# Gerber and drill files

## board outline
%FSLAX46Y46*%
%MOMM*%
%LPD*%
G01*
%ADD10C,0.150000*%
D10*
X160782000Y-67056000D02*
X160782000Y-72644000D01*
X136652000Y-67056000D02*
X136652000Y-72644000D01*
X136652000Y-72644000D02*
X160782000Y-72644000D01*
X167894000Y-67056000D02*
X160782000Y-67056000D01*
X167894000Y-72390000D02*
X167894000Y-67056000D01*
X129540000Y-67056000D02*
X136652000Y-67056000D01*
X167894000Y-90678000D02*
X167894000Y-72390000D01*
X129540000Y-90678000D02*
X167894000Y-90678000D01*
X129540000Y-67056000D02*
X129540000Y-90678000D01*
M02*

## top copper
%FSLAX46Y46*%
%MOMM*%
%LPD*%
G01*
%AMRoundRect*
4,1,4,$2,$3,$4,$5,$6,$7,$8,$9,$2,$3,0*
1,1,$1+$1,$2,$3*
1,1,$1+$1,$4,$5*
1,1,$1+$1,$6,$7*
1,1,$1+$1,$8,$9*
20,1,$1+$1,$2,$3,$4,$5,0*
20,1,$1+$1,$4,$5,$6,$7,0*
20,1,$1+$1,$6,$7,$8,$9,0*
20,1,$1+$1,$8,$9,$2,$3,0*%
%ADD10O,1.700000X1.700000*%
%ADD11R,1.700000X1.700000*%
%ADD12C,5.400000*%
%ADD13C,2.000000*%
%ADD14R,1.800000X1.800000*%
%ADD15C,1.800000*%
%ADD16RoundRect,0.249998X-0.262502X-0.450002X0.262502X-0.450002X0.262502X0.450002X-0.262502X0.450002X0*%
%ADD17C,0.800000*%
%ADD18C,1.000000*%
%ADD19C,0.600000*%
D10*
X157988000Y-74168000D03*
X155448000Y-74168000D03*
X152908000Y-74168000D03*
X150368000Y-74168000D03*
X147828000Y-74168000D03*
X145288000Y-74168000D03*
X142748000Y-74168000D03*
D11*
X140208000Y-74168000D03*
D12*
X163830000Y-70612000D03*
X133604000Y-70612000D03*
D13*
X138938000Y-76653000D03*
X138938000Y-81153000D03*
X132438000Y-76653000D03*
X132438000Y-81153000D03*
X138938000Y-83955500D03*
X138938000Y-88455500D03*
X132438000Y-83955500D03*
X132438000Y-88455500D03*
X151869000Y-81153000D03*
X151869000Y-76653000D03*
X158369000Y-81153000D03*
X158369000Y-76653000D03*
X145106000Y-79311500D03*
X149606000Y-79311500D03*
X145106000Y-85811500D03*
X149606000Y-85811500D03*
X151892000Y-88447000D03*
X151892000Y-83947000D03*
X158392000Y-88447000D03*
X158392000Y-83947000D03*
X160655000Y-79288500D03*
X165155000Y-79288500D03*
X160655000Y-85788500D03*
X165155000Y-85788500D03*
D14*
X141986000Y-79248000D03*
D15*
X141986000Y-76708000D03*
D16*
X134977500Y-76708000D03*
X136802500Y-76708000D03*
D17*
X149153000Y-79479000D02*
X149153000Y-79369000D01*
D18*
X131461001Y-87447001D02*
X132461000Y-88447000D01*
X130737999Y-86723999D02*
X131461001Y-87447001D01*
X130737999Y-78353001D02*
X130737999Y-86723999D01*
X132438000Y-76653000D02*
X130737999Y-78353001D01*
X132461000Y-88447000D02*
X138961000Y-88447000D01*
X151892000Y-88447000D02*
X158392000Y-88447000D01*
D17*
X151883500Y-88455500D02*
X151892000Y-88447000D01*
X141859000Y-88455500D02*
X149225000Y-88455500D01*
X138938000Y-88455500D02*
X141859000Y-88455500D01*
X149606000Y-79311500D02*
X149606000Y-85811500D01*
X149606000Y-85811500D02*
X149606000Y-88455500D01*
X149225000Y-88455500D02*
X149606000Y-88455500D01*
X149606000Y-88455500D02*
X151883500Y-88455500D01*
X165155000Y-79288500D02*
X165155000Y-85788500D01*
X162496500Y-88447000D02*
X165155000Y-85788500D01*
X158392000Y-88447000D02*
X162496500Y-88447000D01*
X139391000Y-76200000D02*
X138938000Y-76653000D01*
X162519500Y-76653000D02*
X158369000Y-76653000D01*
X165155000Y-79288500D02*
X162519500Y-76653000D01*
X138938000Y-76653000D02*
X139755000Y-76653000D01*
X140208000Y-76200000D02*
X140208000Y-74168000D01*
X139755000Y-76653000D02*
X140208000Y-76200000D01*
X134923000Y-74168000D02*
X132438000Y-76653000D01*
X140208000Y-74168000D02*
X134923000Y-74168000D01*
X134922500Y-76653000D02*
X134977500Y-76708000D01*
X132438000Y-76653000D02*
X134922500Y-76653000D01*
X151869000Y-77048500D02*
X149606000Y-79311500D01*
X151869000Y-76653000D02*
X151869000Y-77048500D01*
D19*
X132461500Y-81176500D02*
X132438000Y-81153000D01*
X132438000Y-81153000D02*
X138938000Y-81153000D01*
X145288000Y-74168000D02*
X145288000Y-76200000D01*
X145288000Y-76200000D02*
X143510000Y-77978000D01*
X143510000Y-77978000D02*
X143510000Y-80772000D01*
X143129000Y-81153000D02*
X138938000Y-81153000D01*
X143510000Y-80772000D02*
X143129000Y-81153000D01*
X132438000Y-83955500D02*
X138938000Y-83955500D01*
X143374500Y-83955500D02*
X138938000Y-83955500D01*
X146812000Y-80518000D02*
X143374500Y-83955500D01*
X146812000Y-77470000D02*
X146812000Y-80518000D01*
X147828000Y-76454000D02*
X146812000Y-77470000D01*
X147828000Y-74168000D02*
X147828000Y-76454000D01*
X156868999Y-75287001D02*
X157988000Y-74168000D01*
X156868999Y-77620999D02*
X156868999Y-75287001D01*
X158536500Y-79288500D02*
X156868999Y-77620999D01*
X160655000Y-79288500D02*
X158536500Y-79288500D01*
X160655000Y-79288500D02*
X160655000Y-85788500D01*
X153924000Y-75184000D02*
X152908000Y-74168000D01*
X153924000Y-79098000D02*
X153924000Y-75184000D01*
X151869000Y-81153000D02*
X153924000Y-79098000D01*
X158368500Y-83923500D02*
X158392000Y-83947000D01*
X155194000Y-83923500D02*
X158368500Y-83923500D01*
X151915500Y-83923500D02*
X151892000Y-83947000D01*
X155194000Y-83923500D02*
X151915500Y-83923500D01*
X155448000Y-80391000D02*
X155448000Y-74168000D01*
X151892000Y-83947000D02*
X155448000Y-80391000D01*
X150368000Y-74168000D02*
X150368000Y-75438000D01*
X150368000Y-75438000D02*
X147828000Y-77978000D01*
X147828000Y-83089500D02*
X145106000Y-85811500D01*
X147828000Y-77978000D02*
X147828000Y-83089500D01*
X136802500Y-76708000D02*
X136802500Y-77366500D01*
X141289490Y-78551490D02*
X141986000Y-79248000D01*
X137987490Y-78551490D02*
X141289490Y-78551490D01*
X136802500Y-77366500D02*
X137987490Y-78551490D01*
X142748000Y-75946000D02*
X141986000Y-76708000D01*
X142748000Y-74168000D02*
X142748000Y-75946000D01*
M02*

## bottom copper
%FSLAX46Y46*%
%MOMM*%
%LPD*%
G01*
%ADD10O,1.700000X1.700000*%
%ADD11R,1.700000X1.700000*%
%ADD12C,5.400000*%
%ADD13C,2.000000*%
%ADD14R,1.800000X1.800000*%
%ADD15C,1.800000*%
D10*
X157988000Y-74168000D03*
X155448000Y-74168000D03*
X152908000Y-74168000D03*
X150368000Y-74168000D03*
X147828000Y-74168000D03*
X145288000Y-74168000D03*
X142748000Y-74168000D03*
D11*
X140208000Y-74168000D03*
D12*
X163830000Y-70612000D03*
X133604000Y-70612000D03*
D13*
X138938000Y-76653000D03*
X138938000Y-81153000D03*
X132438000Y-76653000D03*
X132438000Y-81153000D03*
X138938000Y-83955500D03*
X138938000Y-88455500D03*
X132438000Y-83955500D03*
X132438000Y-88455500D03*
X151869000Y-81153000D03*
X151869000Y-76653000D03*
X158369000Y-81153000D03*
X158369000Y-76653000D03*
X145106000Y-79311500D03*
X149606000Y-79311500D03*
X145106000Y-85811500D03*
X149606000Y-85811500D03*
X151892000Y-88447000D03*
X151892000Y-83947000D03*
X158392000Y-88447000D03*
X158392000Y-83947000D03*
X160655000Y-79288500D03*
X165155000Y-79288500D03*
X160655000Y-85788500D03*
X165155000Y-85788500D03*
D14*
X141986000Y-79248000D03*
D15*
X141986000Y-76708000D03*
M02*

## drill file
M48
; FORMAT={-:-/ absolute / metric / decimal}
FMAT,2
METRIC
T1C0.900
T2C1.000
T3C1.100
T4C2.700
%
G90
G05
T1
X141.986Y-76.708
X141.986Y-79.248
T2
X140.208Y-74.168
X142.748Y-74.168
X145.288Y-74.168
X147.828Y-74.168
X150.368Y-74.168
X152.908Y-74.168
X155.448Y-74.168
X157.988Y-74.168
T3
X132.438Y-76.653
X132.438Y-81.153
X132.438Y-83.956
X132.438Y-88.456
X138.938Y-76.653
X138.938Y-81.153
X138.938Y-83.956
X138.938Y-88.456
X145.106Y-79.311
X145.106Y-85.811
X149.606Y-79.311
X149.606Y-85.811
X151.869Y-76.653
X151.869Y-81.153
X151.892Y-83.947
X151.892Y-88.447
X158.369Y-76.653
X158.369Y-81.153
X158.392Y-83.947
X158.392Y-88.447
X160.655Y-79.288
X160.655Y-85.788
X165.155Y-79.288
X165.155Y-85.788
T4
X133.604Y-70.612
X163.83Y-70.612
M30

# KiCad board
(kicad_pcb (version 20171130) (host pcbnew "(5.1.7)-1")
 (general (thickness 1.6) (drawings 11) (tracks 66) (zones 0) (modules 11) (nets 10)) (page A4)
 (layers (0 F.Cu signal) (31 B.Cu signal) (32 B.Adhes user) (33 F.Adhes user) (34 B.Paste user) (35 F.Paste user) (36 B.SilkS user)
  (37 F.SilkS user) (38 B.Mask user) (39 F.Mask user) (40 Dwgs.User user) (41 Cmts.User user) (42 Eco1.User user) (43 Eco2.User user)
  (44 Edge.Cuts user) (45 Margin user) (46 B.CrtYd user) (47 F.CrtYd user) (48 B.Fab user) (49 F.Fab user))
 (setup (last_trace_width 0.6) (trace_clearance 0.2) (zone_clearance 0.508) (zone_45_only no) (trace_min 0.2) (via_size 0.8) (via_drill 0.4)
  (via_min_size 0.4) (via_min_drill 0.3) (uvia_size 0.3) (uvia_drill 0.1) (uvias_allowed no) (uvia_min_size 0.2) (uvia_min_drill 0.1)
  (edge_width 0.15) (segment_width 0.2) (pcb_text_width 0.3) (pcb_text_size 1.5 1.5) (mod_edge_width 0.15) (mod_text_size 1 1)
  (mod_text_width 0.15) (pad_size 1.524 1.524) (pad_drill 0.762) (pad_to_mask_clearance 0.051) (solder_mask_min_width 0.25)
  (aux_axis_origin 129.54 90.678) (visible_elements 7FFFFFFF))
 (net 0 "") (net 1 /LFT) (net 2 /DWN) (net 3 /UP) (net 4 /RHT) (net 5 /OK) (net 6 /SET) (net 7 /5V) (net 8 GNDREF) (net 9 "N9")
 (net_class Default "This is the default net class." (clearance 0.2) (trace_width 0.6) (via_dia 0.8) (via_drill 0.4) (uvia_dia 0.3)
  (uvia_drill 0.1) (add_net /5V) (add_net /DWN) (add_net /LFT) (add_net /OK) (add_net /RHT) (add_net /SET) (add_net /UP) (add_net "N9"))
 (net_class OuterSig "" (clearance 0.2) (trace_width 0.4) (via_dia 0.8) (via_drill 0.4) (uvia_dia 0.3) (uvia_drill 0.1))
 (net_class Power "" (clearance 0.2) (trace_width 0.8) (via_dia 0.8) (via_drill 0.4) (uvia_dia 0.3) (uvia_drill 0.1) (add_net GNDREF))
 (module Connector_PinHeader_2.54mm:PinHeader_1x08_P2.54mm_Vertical (layer F.Cu) (at 140.208 74.168 90)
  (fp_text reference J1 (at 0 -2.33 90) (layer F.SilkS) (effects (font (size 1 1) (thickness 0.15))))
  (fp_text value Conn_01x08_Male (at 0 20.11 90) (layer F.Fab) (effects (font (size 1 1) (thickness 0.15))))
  (pad 8 thru_hole oval (at 0 17.78 90) (size 1.7 1.7) (drill 1) (layers *.Cu *.Mask) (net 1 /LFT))
  (pad 7 thru_hole oval (at 0 15.24 90) (size 1.7 1.7) (drill 1) (layers *.Cu *.Mask) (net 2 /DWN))
  (pad 6 thru_hole oval (at 0 12.7 90) (size 1.7 1.7) (drill 1) (layers *.Cu *.Mask) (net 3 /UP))
  (pad 5 thru_hole oval (at 0 10.16 90) (size 1.7 1.7) (drill 1) (layers *.Cu *.Mask) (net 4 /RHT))
  (pad 4 thru_hole oval (at 0 7.62 90) (size 1.7 1.7) (drill 1) (layers *.Cu *.Mask) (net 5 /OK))
  (pad 3 thru_hole oval (at 0 5.08 90) (size 1.7 1.7) (drill 1) (layers *.Cu *.Mask) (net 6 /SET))
  (pad 2 thru_hole oval (at 0 2.54 90) (size 1.7 1.7) (drill 1) (layers *.Cu *.Mask) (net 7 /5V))
  (pad 1 thru_hole rect (at 0 0 90) (size 1.7 1.7) (drill 1) (layers *.Cu *.Mask) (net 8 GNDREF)))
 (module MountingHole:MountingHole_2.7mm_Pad (layer F.Cu) (at 163.83 70.612)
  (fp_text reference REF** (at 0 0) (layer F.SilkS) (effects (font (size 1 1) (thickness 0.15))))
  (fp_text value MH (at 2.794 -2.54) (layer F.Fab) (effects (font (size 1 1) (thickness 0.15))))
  (pad 1 thru_hole circle (at 0 0) (size 5.4 5.4) (drill 2.7) (layers *.Cu *.Mask)))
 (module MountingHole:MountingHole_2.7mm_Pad (layer F.Cu) (at 133.604 70.612)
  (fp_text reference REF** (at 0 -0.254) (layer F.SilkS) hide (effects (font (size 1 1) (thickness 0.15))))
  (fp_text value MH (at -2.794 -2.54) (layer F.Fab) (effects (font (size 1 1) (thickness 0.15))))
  (pad 1 thru_hole circle (at 0 0) (size 5.4 5.4) (drill 2.7) (layers *.Cu *.Mask)))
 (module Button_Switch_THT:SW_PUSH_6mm (layer F.Cu) (at 132.438 76.653)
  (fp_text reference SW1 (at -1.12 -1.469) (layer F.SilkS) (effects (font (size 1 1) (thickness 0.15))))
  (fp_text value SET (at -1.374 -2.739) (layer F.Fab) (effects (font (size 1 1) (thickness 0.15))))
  (pad 1 thru_hole circle (at 6.5 0 90) (size 2 2) (drill 1.1) (layers *.Cu *.Mask) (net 8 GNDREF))
  (pad 2 thru_hole circle (at 6.5 4.5 90) (size 2 2) (drill 1.1) (layers *.Cu *.Mask) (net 6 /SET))
  (pad 1 thru_hole circle (at 0 0 90) (size 2 2) (drill 1.1) (layers *.Cu *.Mask) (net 8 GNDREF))
  (pad 2 thru_hole circle (at 0 4.5 90) (size 2 2) (drill 1.1) (layers *.Cu *.Mask) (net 6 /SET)))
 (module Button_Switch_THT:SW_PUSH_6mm (layer F.Cu) (at 138.938 88.4555 180)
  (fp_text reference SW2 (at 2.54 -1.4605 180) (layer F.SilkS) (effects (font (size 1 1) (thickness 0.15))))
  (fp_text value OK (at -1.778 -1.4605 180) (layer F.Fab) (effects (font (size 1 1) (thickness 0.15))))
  (pad 2 thru_hole circle (at 0 4.5 270) (size 2 2) (drill 1.1) (layers *.Cu *.Mask) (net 5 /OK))
  (pad 1 thru_hole circle (at 0 0 270) (size 2 2) (drill 1.1) (layers *.Cu *.Mask) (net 8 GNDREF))
  (pad 2 thru_hole circle (at 6.5 4.5 270) (size 2 2) (drill 1.1) (layers *.Cu *.Mask) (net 5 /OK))
  (pad 1 thru_hole circle (at 6.5 0 270) (size 2 2) (drill 1.1) (layers *.Cu *.Mask) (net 8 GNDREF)))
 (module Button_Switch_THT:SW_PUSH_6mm (layer F.Cu) (at 158.369 81.153 180)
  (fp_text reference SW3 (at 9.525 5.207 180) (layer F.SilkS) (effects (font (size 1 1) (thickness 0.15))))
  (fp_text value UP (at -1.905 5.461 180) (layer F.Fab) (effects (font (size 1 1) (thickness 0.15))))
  (pad 1 thru_hole circle (at 6.5 0 270) (size 2 2) (drill 1.1) (layers *.Cu *.Mask) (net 3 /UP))
  (pad 2 thru_hole circle (at 6.5 4.5 270) (size 2 2) (drill 1.1) (layers *.Cu *.Mask) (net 8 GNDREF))
  (pad 1 thru_hole circle (at 0 0 270) (size 2 2) (drill 1.1) (layers *.Cu *.Mask) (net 3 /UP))
  (pad 2 thru_hole circle (at 0 4.5 270) (size 2 2) (drill 1.1) (layers *.Cu *.Mask) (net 8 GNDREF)))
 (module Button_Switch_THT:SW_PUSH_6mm (layer F.Cu) (at 149.606 79.3115 270)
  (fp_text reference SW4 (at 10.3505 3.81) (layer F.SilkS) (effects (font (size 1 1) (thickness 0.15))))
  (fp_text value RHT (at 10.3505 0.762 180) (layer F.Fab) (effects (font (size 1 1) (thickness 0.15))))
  (pad 2 thru_hole circle (at 0 4.5) (size 2 2) (drill 1.1) (layers *.Cu *.Mask) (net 4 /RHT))
  (pad 1 thru_hole circle (at 0 0) (size 2 2) (drill 1.1) (layers *.Cu *.Mask) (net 8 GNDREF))
  (pad 2 thru_hole circle (at 6.5 4.5) (size 2 2) (drill 1.1) (layers *.Cu *.Mask) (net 4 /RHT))
  (pad 1 thru_hole circle (at 6.5 0) (size 2 2) (drill 1.1) (layers *.Cu *.Mask) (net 8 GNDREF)))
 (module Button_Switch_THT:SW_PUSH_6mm (layer F.Cu) (at 151.892 83.947)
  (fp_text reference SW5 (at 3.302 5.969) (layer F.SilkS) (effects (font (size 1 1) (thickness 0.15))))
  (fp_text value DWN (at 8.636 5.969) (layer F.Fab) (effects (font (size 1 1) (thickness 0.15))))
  (pad 2 thru_hole circle (at 0 4.5 90) (size 2 2) (drill 1.1) (layers *.Cu *.Mask) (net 8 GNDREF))
  (pad 1 thru_hole circle (at 0 0 90) (size 2 2) (drill 1.1) (layers *.Cu *.Mask) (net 2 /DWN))
  (pad 2 thru_hole circle (at 6.5 4.5 90) (size 2 2) (drill 1.1) (layers *.Cu *.Mask) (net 8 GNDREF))
  (pad 1 thru_hole circle (at 6.5 0 90) (size 2 2) (drill 1.1) (layers *.Cu *.Mask) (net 2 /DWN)))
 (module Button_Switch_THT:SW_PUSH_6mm (layer F.Cu) (at 160.655 85.7885 90)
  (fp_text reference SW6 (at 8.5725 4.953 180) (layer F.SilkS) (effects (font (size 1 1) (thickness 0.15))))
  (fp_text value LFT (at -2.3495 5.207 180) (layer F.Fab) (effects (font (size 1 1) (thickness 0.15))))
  (pad 1 thru_hole circle (at 6.5 0 180) (size 2 2) (drill 1.1) (layers *.Cu *.Mask) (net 1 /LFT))
  (pad 2 thru_hole circle (at 6.5 4.5 180) (size 2 2) (drill 1.1) (layers *.Cu *.Mask) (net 8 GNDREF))
  (pad 1 thru_hole circle (at 0 0 180) (size 2 2) (drill 1.1) (layers *.Cu *.Mask) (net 1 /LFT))
  (pad 2 thru_hole circle (at 0 4.5 180) (size 2 2) (drill 1.1) (layers *.Cu *.Mask) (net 8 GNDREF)))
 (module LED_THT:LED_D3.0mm (layer F.Cu) (at 141.986 79.248 90)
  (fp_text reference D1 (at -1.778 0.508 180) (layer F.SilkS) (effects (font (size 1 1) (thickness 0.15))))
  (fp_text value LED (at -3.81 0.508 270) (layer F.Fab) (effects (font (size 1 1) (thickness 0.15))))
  (pad 1 thru_hole rect (at 0 0 90) (size 1.8 1.8) (drill 0.9) (layers *.Cu *.Mask) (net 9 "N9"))
  (pad 2 thru_hole circle (at 2.54 0 90) (size 1.8 1.8) (drill 0.9) (layers *.Cu *.Mask) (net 7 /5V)))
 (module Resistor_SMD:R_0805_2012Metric (layer F.Cu) (at 135.89 76.708)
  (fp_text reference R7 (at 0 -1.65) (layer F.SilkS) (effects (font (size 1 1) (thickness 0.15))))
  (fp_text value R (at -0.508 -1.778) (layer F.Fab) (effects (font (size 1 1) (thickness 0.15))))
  (pad 1 smd roundrect (at -0.9125 0) (size 1.025 1.4) (layers F.Cu F.Paste F.Mask) (roundrect_rratio 0.2439004878048781) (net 8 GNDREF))
  (pad 2 smd roundrect (at 0.9125 0) (size 1.025 1.4) (layers F.Cu F.Paste F.Mask) (roundrect_rratio 0.2439004878048781) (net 9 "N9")))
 (gr_line (start 160.782 67.056) (end 160.782 72.644) (layer Edge.Cuts) (width 0.15))
 (gr_line (start 136.652 67.056) (end 136.652 72.644) (layer Edge.Cuts) (width 0.15))
 (gr_line (start 136.652 72.644) (end 160.782 72.644) (layer Edge.Cuts) (width 0.15))
 (gr_line (start 167.894 67.056) (end 160.782 67.056) (layer Edge.Cuts) (width 0.15))
 (gr_line (start 167.894 72.39) (end 167.894 67.056) (layer Edge.Cuts) (width 0.15))
 (gr_line (start 129.54 67.056) (end 136.652 67.056) (layer Edge.Cuts) (width 0.15))
 (gr_line (start 167.894 90.678) (end 167.894 72.39) (layer Edge.Cuts) (width 0.15))
 (gr_line (start 129.54 90.678) (end 167.894 90.678) (layer Edge.Cuts) (width 0.15))
 (gr_line (start 129.54 67.056) (end 129.54 90.678) (layer Edge.Cuts) (width 0.15))
 (segment (start 149.153 79.479) (end 149.153 79.369) (width 0.8) (layer F.Cu) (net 8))
 (segment (start 131.461001 87.447001) (end 132.461 88.447) (width 1) (layer F.Cu) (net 8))
 (segment (start 130.737999 86.723999) (end 131.461001 87.447001) (width 1) (layer F.Cu) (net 8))
 (segment (start 130.737999 78.353001) (end 130.737999 86.723999) (width 1) (layer F.Cu) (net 8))
 (segment (start 132.438 76.653) (end 130.737999 78.353001) (width 1) (layer F.Cu) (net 8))
 (segment (start 132.461 88.447) (end 138.961 88.447) (width 1) (layer F.Cu) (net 8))
 (segment (start 151.892 88.447) (end 158.392 88.447) (width 1) (layer F.Cu) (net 8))
 (segment (start 151.8835 88.4555) (end 151.892 88.447) (width 0.8) (layer F.Cu) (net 8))
 (segment (start 141.859 88.4555) (end 149.225 88.4555) (width 0.8) (layer F.Cu) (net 8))
 (segment (start 138.938 88.4555) (end 141.859 88.4555) (width 0.8) (layer F.Cu) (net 8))
 (segment (start 149.606 79.3115) (end 149.606 85.8115) (width 0.8) (layer F.Cu) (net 8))
 (segment (start 149.606 85.8115) (end 149.606 88.4555) (width 0.8) (layer F.Cu) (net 8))
 (segment (start 149.225 88.4555) (end 149.606 88.4555) (width 0.8) (layer F.Cu) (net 8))
 (segment (start 149.606 88.4555) (end 151.8835 88.4555) (width 0.8) (layer F.Cu) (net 8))
 (segment (start 165.155 79.2885) (end 165.155 85.7885) (width 0.8) (layer F.Cu) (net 8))
 (segment (start 162.4965 88.447) (end 165.155 85.7885) (width 0.8) (layer F.Cu) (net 8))
 (segment (start 158.392 88.447) (end 162.4965 88.447) (width 0.8) (layer F.Cu) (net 8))
 (segment (start 139.391 76.2) (end 138.938 76.653) (width 0.8) (layer F.Cu) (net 8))
 (segment (start 162.5195 76.653) (end 158.369 76.653) (width 0.8) (layer F.Cu) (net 8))
 (segment (start 165.155 79.2885) (end 162.5195 76.653) (width 0.8) (layer F.Cu) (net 8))
 (segment (start 138.938 76.653) (end 139.755 76.653) (width 0.8) (layer F.Cu) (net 8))
 (segment (start 140.208 76.2) (end 140.208 74.168) (width 0.8) (layer F.Cu) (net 8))
 (segment (start 139.755 76.653) (end 140.208 76.2) (width 0.8) (layer F.Cu) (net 8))
 (segment (start 134.923 74.168) (end 132.438 76.653) (width 0.8) (layer F.Cu) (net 8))
 (segment (start 140.208 74.168) (end 134.923 74.168) (width 0.8) (layer F.Cu) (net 8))
 (segment (start 134.9225 76.653) (end 134.9775 76.708) (width 0.8) (layer F.Cu) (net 8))
 (segment (start 132.438 76.653) (end 134.9225 76.653) (width 0.8) (layer F.Cu) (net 8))
 (segment (start 151.869 77.0485) (end 149.606 79.3115) (width 0.8) (layer F.Cu) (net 8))
 (segment (start 151.869 76.653) (end 151.869 77.0485) (width 0.8) (layer F.Cu) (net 8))
 (segment (start 132.4615 81.1765) (end 132.438 81.153) (width 0.6) (layer F.Cu) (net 6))
 (segment (start 132.438 81.153) (end 138.938 81.153) (width 0.6) (layer F.Cu) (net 6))
 (segment (start 145.288 74.168) (end 145.288 76.2) (width 0.6) (layer F.Cu) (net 6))
 (segment (start 145.288 76.2) (end 143.51 77.978) (width 0.6) (layer F.Cu) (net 6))
 (segment (start 143.51 77.978) (end 143.51 80.772) (width 0.6) (layer F.Cu) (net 6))
 (segment (start 143.129 81.153) (end 138.938 81.153) (width 0.6) (layer F.Cu) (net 6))
 (segment (start 143.51 80.772) (end 143.129 81.153) (width 0.6) (layer F.Cu) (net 6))
 (segment (start 132.438 83.9555) (end 138.938 83.9555) (width 0.6) (layer F.Cu) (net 5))
 (segment (start 143.3745 83.9555) (end 138.938 83.9555) (width 0.6) (layer F.Cu) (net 5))
 (segment (start 146.812 80.518) (end 143.3745 83.9555) (width 0.6) (layer F.Cu) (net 5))
 (segment (start 146.812 77.47) (end 146.812 80.518) (width 0.6) (layer F.Cu) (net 5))
 (segment (start 147.828 76.454) (end 146.812 77.47) (width 0.6) (layer F.Cu) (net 5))
 (segment (start 147.828 74.168) (end 147.828 76.454) (width 0.6) (layer F.Cu) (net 5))
 (segment (start 156.868999 75.287001) (end 157.988 74.168) (width 0.6) (layer F.Cu) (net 1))
 (segment (start 156.868999 77.620999) (end 156.868999 75.287001) (width 0.6) (layer F.Cu) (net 1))
 (segment (start 158.5365 79.2885) (end 156.868999 77.620999) (width 0.6) (layer F.Cu) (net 1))
 (segment (start 160.655 79.2885) (end 158.5365 79.2885) (width 0.6) (layer F.Cu) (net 1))
 (segment (start 160.655 79.2885) (end 160.655 85.7885) (width 0.6) (layer F.Cu) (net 1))
 (segment (start 153.924 75.184) (end 152.908 74.168) (width 0.6) (layer F.Cu) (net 3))
 (segment (start 153.924 79.098) (end 153.924 75.184) (width 0.6) (layer F.Cu) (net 3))
 (segment (start 151.869 81.153) (end 153.924 79.098) (width 0.6) (layer F.Cu) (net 3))
 (segment (start 158.3685 83.9235) (end 158.392 83.947) (width 0.6) (layer F.Cu) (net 2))
 (segment (start 155.194 83.9235) (end 158.3685 83.9235) (width 0.6) (layer F.Cu) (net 2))
 (segment (start 151.9155 83.9235) (end 151.892 83.947) (width 0.6) (layer F.Cu) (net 2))
 (segment (start 155.194 83.9235) (end 151.9155 83.9235) (width 0.6) (layer F.Cu) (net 2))
 (segment (start 155.448 80.391) (end 155.448 74.168) (width 0.6) (layer F.Cu) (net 2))
 (segment (start 151.892 83.947) (end 155.448 80.391) (width 0.6) (layer F.Cu) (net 2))
 (segment (start 150.368 74.168) (end 150.368 75.438) (width 0.6) (layer F.Cu) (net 4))
 (segment (start 150.368 75.438) (end 147.828 77.978) (width 0.6) (layer F.Cu) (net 4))
 (segment (start 147.828 83.0895) (end 145.106 85.8115) (width 0.6) (layer F.Cu) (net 4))
 (segment (start 147.828 77.978) (end 147.828 83.0895) (width 0.6) (layer F.Cu) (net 4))
 (segment (start 136.8025 76.708) (end 136.8025 77.3665) (width 0.6) (layer F.Cu) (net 9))
 (segment (start 141.28949 78.55149) (end 141.986 79.248) (width 0.6) (layer F.Cu) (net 9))
 (segment (start 137.98749 78.55149) (end 141.28949 78.55149) (width 0.6) (layer F.Cu) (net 9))
 (segment (start 136.8025 77.3665) (end 137.98749 78.55149) (width 0.6) (layer F.Cu) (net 9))
 (segment (start 142.748 75.946) (end 141.986 76.708) (width 0.6) (layer F.Cu) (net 7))
 (segment (start 142.748 74.168) (end 142.748 75.946) (width 0.6) (layer F.Cu) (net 7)))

